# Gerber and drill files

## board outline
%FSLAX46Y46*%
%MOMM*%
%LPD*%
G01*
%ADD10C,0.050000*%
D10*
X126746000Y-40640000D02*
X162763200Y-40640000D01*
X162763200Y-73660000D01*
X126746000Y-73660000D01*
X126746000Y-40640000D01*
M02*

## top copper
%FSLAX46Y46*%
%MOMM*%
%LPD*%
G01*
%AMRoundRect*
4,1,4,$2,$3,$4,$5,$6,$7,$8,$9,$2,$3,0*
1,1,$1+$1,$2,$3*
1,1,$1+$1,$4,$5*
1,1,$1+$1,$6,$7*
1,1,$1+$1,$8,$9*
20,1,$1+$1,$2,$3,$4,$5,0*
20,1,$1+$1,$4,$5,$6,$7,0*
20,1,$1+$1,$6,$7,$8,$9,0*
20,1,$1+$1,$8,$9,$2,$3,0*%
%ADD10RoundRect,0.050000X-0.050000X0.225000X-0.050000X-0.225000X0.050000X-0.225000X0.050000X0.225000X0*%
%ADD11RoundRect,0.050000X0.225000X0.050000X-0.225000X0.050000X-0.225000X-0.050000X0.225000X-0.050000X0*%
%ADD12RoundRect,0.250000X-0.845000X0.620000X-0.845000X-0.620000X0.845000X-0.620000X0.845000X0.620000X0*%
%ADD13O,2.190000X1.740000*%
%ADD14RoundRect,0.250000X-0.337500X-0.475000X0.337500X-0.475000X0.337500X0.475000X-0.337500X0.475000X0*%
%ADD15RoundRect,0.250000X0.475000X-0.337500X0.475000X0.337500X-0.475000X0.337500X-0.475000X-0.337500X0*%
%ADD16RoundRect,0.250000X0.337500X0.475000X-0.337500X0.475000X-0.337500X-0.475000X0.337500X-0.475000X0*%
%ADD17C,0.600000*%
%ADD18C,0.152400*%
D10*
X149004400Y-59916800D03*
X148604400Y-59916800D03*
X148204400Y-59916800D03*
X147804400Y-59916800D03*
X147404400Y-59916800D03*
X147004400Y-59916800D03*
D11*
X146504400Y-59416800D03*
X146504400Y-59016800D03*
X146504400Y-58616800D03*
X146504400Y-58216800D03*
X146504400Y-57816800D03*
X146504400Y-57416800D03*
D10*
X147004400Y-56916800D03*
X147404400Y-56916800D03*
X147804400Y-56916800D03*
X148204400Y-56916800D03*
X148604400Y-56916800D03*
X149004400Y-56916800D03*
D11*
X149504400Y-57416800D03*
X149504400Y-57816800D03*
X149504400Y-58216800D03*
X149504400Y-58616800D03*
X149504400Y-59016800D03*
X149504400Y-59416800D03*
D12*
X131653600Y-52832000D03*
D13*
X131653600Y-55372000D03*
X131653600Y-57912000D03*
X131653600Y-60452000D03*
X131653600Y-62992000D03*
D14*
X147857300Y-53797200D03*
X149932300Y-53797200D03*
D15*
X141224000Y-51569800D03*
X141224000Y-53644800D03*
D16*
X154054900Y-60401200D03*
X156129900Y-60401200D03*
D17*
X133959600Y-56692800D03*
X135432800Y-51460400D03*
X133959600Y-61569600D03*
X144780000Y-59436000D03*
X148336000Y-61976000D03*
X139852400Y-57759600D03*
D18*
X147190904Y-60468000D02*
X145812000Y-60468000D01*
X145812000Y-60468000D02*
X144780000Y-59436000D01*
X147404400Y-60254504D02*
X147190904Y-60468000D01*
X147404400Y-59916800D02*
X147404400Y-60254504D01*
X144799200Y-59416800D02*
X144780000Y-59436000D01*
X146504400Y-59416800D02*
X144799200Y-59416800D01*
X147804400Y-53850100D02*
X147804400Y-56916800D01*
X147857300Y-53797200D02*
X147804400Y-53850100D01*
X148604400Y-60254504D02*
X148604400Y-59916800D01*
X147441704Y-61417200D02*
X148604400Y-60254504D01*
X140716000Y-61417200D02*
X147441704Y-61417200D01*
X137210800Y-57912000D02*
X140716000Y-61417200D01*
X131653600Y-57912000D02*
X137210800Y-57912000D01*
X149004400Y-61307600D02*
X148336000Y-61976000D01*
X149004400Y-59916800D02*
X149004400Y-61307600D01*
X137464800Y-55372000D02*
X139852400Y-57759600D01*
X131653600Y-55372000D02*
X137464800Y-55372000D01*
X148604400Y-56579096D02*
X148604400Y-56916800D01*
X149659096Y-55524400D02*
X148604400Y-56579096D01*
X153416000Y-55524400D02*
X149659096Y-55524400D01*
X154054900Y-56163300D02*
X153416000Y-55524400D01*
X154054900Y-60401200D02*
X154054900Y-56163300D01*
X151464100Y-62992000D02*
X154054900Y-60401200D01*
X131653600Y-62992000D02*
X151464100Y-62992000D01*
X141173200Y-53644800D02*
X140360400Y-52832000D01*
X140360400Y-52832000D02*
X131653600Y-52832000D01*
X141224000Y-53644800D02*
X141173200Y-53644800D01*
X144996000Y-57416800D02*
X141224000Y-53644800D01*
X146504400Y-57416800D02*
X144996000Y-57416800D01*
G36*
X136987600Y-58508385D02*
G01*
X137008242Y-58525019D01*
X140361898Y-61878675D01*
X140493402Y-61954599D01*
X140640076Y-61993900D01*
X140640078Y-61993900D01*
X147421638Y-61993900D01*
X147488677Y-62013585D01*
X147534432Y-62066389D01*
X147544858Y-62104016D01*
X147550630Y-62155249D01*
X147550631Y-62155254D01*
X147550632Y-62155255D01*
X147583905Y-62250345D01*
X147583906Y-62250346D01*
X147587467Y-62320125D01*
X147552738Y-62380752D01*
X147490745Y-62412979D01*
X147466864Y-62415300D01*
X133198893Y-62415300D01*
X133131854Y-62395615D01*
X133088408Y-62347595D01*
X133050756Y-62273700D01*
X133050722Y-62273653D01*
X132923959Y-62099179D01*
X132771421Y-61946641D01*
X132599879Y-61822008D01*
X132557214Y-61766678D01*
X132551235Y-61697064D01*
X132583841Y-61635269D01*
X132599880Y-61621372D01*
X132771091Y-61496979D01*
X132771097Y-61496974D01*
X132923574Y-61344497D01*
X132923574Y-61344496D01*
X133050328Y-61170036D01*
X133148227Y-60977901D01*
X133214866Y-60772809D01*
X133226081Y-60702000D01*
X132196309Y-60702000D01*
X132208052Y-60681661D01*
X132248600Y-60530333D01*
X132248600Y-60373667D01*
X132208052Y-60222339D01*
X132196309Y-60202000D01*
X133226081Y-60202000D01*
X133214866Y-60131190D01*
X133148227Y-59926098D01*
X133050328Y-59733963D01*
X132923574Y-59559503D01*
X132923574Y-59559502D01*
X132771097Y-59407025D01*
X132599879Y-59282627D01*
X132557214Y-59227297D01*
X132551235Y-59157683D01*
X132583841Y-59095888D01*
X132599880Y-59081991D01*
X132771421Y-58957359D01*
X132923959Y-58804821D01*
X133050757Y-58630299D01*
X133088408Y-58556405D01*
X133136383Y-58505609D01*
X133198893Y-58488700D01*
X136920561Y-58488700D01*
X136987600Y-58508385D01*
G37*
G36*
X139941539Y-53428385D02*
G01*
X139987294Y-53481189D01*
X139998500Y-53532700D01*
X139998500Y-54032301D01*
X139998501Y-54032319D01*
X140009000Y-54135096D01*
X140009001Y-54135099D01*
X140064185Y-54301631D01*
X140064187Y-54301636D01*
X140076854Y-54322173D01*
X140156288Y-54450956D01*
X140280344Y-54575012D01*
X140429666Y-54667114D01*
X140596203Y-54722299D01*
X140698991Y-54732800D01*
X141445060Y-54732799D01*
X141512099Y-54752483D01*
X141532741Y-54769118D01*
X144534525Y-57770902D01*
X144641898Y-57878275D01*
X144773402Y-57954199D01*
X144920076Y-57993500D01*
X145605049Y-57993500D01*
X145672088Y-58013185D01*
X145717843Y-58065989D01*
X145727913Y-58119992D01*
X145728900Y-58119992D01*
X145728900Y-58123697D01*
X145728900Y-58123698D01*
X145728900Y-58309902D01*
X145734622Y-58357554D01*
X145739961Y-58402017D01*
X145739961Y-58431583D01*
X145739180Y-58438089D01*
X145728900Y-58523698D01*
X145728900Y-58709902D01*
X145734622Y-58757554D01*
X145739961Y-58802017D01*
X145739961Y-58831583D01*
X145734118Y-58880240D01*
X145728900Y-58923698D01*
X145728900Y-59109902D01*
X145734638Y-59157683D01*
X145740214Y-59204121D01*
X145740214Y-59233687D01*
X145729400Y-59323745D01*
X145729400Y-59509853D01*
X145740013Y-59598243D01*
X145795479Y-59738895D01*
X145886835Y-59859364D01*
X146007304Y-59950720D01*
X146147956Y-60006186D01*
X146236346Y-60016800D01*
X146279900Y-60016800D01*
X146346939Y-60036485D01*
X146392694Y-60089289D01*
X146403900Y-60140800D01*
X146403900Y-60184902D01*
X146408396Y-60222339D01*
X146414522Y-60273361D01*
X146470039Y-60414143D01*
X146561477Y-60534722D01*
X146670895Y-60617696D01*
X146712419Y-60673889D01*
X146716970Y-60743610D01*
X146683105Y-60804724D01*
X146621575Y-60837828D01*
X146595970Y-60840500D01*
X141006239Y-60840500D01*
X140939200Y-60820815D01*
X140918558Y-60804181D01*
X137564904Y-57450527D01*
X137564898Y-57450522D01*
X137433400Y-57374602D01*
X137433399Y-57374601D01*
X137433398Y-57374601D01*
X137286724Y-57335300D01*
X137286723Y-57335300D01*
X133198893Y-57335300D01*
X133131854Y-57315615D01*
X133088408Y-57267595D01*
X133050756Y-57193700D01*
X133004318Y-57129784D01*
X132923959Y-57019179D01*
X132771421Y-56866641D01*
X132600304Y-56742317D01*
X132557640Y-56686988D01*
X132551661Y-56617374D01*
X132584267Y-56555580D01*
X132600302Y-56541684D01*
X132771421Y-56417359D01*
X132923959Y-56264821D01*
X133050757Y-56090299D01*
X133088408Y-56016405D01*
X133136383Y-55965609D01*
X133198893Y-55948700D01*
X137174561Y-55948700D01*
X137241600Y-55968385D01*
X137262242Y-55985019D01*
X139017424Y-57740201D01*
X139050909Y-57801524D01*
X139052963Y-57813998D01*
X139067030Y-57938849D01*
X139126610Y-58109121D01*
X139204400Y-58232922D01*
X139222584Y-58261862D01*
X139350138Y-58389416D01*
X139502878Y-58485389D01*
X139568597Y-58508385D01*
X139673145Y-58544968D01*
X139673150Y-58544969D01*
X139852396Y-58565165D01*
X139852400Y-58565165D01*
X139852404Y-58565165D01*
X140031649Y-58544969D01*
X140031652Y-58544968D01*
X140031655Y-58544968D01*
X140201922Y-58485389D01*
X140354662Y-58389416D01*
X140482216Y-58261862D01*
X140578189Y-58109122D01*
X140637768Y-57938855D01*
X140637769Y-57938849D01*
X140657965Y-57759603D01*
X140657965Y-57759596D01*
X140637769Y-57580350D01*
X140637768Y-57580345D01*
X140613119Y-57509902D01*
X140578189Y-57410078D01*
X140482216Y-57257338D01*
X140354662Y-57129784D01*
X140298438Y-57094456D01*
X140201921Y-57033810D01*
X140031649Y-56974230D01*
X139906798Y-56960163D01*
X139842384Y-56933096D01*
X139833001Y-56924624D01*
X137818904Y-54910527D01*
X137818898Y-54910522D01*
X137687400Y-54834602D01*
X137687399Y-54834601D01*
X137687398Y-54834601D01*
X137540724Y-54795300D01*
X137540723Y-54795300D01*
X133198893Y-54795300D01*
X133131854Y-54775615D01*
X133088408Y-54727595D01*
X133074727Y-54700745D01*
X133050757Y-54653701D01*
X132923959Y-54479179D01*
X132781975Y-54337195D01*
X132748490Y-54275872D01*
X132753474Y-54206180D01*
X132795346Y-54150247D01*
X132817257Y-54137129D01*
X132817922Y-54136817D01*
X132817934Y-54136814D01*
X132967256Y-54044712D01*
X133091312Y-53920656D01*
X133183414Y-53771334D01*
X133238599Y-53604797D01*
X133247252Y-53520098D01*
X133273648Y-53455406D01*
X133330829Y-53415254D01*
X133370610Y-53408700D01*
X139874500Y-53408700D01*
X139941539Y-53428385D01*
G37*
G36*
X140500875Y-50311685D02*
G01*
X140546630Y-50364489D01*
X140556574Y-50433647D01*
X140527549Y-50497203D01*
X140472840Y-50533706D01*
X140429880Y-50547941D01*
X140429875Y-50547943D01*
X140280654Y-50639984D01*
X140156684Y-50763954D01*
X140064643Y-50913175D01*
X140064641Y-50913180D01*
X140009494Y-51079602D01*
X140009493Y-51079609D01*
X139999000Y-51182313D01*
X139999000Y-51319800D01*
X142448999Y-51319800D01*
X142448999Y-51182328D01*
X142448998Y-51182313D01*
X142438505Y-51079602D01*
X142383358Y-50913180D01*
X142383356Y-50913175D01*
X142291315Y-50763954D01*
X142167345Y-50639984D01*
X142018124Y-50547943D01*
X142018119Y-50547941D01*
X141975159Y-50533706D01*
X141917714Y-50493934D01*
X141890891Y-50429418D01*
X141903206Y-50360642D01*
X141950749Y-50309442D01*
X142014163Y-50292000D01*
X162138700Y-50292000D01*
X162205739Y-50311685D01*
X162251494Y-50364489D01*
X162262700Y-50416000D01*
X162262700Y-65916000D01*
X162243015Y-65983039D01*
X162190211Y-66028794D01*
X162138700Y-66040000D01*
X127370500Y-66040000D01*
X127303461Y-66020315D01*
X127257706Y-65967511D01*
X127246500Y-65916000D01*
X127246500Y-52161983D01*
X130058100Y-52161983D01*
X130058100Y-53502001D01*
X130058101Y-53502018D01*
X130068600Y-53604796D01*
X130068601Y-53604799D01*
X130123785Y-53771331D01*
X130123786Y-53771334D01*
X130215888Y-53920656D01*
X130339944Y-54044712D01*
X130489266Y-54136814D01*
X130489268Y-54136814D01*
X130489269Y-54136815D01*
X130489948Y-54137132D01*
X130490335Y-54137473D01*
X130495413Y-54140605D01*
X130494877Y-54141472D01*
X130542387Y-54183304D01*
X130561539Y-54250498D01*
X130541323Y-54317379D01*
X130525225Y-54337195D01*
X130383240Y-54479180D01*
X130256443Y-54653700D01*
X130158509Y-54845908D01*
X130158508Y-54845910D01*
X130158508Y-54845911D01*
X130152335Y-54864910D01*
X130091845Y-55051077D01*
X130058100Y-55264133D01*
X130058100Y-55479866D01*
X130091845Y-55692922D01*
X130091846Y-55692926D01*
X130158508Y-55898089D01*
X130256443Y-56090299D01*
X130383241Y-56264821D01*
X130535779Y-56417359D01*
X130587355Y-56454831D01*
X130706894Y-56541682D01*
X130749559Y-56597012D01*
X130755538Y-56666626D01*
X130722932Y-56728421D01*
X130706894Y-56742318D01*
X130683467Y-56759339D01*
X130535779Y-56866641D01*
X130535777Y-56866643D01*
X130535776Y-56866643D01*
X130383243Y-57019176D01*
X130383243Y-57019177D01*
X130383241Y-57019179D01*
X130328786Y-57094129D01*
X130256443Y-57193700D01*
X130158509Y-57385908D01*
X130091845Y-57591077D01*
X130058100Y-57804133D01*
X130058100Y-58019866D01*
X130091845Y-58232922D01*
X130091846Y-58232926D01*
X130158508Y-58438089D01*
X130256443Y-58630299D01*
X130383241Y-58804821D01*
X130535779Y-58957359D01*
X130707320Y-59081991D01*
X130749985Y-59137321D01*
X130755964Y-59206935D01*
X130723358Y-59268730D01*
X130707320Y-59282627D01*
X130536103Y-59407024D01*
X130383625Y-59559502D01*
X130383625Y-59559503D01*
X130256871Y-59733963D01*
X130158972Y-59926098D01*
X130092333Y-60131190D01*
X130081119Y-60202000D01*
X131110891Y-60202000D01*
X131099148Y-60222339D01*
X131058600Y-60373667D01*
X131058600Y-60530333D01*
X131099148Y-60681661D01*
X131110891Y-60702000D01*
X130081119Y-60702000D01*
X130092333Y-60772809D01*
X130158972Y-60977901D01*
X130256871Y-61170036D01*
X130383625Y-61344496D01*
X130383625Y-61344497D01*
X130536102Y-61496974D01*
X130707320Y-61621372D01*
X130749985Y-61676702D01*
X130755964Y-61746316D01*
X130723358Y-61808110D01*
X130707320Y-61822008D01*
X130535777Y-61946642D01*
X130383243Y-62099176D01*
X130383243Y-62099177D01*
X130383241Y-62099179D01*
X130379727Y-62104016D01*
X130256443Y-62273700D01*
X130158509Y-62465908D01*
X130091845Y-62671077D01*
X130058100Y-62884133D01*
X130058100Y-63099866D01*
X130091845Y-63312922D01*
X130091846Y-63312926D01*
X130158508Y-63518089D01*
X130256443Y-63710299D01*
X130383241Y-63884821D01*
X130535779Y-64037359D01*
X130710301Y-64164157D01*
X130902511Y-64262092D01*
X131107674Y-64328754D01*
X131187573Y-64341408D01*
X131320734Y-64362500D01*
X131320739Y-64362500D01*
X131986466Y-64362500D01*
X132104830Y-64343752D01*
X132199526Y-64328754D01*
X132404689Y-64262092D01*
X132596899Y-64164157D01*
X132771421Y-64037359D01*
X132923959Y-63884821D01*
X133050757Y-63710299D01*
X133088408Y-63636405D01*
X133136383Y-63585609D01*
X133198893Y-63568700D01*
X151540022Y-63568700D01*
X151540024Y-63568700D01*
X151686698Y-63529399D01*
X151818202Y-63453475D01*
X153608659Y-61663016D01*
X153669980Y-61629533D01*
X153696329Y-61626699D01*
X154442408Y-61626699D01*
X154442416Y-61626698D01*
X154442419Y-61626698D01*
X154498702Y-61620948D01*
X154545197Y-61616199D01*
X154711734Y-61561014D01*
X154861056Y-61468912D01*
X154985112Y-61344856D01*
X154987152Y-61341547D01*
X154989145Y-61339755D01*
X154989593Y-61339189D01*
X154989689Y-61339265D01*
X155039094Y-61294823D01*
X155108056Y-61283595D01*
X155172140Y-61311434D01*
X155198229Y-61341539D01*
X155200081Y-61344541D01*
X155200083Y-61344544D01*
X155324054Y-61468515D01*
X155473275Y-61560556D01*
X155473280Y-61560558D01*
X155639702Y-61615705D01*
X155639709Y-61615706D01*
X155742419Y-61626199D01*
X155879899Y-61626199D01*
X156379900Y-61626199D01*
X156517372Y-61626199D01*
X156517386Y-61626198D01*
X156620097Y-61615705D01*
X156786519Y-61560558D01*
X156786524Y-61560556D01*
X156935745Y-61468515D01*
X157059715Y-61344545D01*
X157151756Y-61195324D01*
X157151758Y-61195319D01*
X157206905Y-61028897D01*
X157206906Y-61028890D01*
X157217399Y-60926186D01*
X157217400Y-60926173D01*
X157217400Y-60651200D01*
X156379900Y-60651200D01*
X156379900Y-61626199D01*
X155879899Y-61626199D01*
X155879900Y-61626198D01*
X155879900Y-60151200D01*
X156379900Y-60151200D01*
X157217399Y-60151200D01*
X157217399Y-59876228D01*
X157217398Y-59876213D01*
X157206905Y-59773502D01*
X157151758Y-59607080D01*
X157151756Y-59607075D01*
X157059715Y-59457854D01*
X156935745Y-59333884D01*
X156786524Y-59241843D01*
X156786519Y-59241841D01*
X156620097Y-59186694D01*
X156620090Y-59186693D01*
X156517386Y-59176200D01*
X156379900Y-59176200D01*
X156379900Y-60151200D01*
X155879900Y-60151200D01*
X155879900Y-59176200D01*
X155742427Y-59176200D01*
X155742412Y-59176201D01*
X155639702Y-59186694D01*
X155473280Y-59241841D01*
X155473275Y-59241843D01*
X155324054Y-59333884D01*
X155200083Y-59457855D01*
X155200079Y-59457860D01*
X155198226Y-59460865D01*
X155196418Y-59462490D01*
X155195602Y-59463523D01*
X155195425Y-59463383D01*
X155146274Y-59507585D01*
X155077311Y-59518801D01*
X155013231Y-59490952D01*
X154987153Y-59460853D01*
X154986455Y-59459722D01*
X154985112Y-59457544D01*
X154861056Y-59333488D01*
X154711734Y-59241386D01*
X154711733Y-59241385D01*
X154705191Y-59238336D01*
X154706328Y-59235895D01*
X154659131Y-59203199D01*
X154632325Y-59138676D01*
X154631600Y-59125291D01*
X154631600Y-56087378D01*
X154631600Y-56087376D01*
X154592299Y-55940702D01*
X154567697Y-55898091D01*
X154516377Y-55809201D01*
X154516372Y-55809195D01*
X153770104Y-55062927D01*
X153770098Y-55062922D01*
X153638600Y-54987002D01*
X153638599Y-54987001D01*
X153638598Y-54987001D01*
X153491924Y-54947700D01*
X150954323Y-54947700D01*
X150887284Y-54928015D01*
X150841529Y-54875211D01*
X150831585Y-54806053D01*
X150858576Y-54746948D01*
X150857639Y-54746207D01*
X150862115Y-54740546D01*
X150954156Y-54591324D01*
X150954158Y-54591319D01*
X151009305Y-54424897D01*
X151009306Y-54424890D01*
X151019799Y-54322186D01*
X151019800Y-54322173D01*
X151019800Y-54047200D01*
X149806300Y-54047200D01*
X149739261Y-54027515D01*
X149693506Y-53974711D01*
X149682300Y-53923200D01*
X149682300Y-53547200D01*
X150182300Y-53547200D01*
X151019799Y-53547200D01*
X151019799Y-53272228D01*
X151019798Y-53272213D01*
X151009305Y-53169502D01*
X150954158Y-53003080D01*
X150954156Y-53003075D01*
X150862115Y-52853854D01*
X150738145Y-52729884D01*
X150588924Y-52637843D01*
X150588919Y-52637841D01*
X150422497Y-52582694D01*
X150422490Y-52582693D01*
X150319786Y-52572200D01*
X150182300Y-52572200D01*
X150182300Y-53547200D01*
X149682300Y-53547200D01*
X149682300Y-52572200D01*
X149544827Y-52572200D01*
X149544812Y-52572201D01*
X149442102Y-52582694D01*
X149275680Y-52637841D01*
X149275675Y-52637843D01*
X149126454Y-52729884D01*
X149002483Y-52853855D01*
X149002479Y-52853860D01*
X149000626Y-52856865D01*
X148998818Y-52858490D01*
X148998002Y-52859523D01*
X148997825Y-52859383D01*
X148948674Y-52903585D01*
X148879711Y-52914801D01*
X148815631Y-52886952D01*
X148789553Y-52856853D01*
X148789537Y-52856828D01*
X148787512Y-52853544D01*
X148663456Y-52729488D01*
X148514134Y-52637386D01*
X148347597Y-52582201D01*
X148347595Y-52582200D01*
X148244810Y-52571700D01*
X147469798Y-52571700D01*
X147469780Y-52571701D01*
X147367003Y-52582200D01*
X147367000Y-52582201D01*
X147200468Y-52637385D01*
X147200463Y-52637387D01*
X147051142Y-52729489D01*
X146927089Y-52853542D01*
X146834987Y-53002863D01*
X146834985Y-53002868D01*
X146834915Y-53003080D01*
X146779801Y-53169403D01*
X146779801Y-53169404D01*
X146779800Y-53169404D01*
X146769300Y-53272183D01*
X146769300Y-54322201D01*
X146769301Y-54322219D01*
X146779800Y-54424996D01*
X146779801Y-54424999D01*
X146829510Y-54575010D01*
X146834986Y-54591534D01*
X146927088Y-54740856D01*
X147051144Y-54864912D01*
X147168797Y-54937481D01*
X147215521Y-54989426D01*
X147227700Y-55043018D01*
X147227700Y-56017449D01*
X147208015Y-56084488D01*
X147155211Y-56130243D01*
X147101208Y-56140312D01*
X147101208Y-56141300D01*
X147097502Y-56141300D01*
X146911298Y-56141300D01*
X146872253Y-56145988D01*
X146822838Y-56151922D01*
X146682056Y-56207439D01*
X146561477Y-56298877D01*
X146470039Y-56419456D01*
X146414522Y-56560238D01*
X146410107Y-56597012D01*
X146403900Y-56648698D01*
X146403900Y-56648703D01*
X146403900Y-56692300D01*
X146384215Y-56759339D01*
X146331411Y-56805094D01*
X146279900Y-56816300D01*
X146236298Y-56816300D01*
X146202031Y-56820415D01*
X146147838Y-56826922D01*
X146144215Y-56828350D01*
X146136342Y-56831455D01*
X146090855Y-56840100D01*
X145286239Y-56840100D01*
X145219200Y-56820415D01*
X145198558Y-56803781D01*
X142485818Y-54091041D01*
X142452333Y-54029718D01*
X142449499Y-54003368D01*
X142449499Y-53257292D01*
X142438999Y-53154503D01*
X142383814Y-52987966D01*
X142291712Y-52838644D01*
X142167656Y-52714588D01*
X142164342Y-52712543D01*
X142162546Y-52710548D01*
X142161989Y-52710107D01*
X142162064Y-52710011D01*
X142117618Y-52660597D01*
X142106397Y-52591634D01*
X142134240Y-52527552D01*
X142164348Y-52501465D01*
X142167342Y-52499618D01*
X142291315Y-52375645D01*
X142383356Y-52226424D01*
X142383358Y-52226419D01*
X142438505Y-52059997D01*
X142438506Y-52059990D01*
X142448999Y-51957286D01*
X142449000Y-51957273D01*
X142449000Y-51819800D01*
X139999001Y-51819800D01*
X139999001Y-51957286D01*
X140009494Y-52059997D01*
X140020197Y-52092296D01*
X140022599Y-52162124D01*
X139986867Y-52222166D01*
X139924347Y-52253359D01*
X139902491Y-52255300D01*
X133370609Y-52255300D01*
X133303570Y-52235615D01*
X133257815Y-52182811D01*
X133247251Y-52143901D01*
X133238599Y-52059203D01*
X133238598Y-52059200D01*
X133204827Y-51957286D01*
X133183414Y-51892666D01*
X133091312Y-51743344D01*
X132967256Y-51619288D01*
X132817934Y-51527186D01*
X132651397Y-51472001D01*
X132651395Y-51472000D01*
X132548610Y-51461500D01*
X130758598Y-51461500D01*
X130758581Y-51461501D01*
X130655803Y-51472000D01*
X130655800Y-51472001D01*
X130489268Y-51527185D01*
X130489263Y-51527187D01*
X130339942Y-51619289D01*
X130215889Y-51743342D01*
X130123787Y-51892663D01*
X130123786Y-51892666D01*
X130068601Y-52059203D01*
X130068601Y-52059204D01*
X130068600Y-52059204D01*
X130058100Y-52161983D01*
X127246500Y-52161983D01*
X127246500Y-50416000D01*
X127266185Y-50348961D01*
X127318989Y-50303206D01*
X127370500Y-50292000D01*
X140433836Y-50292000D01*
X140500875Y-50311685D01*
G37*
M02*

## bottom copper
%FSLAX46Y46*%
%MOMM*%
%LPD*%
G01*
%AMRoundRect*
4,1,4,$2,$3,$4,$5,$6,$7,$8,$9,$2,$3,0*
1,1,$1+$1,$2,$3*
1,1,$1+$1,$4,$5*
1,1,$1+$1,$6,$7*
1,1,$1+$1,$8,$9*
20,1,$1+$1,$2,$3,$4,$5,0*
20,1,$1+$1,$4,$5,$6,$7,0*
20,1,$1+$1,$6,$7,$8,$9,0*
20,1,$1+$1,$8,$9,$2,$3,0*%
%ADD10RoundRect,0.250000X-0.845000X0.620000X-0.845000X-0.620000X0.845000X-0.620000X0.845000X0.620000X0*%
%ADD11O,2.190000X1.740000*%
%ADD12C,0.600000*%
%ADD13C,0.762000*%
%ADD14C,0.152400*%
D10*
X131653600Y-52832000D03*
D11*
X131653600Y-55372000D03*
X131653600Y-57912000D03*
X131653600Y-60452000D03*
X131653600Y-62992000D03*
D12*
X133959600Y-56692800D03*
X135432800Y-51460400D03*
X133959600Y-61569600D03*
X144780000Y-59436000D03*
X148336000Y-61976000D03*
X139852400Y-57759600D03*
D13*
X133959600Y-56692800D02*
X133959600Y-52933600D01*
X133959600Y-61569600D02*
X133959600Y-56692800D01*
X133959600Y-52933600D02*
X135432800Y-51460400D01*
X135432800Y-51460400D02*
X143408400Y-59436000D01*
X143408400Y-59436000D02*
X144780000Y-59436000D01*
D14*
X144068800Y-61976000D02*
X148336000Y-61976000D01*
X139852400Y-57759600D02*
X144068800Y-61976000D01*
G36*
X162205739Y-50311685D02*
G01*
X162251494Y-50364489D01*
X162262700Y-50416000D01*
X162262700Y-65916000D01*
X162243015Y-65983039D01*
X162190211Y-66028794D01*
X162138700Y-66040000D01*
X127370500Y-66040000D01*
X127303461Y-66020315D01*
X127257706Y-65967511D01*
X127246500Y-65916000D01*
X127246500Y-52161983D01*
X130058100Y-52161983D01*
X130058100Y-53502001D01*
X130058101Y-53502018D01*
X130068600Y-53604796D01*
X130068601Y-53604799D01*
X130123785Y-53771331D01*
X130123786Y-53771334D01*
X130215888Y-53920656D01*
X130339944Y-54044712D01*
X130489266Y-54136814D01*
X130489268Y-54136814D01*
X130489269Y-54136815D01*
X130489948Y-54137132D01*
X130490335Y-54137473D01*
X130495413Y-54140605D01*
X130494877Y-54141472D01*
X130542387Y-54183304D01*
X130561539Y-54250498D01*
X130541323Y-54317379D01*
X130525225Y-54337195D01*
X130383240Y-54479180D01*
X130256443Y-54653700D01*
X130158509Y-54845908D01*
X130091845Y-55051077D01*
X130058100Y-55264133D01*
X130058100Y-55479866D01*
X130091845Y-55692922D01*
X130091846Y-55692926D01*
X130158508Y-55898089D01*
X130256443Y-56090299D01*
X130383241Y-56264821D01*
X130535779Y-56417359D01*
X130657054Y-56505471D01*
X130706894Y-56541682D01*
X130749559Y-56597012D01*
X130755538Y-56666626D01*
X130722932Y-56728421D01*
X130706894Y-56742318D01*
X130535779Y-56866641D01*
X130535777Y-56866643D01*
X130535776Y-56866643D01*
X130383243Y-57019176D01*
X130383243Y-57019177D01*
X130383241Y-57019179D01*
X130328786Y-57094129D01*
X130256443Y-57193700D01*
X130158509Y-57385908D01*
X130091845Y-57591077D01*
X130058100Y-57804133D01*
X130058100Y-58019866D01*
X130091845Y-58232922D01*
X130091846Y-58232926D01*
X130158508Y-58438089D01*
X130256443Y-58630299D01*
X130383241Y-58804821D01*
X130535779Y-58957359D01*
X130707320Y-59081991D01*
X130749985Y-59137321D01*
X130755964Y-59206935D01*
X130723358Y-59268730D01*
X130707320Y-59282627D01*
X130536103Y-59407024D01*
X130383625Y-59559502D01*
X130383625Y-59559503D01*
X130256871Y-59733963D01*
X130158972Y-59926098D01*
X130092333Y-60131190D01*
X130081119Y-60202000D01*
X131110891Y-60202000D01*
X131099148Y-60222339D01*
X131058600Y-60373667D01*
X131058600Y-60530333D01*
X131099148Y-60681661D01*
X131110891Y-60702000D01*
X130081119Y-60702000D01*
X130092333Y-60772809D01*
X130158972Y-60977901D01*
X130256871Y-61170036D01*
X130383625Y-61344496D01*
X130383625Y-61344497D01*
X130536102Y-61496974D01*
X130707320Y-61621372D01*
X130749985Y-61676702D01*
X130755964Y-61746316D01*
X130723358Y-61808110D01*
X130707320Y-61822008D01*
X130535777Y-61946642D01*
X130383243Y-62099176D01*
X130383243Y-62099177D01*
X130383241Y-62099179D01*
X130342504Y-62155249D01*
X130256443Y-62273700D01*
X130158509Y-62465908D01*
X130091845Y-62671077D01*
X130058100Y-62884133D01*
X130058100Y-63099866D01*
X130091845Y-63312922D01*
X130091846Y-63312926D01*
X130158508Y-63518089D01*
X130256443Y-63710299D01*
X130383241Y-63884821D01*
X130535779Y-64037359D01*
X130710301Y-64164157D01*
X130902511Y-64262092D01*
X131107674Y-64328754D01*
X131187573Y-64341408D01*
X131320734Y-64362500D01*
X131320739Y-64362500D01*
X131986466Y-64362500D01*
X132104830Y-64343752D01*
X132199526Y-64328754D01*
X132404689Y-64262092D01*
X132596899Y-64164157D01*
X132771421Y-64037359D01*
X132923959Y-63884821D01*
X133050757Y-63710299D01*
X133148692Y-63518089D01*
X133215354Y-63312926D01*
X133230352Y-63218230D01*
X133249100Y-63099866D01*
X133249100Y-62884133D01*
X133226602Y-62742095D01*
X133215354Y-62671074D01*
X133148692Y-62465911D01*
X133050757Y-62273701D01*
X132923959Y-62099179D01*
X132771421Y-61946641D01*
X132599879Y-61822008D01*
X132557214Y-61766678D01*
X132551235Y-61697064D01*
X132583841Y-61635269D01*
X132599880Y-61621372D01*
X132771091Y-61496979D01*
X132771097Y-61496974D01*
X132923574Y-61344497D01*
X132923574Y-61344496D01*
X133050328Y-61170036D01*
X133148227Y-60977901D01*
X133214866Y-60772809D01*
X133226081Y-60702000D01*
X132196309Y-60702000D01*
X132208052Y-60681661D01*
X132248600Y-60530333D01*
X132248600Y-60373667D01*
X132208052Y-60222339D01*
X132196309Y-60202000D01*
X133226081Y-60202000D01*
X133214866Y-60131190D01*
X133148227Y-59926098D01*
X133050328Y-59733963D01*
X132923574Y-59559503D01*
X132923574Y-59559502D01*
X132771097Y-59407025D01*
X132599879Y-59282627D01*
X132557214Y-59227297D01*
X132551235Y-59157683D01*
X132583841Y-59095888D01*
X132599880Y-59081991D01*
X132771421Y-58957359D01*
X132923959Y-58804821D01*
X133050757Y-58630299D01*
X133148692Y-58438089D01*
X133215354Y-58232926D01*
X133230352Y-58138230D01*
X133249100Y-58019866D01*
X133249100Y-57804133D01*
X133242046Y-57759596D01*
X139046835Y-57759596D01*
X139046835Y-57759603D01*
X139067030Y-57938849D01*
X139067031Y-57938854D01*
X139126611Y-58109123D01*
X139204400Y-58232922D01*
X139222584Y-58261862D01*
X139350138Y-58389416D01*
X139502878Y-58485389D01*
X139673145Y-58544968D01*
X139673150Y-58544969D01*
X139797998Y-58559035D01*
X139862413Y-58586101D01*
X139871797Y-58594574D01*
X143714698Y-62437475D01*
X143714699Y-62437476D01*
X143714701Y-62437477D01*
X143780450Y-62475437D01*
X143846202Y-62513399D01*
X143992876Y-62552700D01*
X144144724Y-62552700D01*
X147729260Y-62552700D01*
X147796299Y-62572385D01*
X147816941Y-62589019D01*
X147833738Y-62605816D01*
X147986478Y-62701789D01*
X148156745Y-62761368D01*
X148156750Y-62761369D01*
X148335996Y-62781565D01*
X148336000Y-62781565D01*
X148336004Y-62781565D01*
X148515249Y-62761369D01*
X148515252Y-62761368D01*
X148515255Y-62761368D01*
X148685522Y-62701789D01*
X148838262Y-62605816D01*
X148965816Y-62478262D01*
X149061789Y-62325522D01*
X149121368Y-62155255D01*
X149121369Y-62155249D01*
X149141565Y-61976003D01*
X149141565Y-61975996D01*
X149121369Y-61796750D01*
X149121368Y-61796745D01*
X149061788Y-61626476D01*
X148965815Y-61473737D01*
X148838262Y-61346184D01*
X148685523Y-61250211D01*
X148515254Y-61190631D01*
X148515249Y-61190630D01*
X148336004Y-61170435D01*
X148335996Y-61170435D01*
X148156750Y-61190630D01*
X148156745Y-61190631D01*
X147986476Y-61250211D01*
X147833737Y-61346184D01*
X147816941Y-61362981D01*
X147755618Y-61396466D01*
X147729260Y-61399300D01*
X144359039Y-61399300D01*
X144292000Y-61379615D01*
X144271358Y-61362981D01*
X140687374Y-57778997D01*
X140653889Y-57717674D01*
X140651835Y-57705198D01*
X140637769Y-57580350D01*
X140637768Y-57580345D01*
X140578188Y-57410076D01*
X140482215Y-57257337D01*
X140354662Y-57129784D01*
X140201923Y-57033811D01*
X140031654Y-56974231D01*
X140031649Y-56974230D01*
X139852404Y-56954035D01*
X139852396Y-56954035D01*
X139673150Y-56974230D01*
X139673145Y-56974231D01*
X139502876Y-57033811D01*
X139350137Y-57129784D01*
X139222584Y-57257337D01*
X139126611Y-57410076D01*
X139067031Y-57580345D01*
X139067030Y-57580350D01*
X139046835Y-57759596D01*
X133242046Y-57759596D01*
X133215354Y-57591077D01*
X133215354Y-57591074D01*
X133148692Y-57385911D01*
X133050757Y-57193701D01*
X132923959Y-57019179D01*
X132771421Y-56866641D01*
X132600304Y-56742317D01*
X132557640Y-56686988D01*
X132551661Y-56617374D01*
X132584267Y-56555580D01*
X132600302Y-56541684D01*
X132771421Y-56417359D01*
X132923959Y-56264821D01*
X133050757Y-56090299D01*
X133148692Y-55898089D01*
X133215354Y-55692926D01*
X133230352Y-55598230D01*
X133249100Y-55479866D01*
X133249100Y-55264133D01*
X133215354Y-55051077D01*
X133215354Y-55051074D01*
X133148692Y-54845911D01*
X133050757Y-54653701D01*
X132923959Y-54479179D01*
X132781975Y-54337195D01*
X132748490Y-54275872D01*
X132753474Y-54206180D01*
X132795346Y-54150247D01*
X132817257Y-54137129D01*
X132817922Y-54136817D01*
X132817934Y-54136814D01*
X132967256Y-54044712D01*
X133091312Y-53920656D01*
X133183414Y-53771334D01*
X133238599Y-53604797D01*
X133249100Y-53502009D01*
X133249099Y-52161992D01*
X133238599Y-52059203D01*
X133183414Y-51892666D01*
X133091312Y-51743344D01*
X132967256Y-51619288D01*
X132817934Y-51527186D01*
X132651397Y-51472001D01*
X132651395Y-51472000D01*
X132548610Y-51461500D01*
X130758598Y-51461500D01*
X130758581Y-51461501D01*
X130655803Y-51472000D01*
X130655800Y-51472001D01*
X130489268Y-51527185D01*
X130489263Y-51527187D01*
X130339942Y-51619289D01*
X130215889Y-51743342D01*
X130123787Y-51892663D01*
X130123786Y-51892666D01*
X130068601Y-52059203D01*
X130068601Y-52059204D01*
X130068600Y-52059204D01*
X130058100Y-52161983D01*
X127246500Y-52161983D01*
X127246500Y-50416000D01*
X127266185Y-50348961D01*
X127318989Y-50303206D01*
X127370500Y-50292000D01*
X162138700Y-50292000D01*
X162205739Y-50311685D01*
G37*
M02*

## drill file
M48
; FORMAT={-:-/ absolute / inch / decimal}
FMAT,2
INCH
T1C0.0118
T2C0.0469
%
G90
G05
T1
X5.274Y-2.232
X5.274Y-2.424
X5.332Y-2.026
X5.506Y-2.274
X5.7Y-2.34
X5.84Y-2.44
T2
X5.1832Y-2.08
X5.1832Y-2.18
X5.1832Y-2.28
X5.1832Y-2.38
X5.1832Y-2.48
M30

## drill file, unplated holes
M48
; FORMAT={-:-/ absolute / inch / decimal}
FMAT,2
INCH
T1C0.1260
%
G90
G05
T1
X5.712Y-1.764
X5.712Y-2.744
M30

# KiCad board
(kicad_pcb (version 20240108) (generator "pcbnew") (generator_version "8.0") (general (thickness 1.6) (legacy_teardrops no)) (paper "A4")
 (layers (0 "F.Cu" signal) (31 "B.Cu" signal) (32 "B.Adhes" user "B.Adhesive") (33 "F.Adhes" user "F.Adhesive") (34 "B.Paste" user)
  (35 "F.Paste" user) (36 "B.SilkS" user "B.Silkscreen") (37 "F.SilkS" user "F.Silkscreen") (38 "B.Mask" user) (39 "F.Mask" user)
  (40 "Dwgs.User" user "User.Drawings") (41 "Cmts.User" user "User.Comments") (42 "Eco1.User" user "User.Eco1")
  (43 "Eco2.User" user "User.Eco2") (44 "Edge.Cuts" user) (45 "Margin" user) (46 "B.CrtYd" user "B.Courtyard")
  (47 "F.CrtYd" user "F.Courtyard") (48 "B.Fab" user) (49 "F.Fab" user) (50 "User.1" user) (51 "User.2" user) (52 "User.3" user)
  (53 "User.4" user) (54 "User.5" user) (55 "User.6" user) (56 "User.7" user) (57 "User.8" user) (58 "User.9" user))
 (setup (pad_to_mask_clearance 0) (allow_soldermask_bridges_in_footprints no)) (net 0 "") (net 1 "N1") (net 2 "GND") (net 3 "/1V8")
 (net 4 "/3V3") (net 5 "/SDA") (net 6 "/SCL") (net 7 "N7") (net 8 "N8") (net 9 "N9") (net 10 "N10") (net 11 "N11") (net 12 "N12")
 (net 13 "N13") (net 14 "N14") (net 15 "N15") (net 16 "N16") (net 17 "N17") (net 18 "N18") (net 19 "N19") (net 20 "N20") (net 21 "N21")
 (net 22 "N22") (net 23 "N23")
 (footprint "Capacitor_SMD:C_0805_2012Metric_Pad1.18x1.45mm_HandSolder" (layer "F.Cu") (at 148.8948 53.7972)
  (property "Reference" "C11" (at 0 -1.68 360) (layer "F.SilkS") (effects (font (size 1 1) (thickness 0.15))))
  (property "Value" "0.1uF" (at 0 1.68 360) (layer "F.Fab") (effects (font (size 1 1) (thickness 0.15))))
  (pad "1" smd roundrect (at -1.0375 0) (size 1.175 1.45) (layers "F.Cu" "F.Paste" "F.Mask") (roundrect_rratio 0.212766) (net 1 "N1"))
  (pad "2" smd roundrect (at 1.0375 0) (size 1.175 1.45) (layers "F.Cu" "F.Paste" "F.Mask") (roundrect_rratio 0.212766) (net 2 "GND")))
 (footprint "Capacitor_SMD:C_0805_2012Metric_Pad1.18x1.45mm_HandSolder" (layer "F.Cu") (at 155.0924 60.4012 180)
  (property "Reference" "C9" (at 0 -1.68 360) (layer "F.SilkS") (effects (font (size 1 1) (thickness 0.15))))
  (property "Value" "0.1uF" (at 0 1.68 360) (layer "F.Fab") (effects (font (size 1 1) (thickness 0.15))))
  (pad "1" smd roundrect (at -1.0375 0 180) (size 1.175 1.45) (layers "F.Cu" "F.Paste" "F.Mask") (roundrect_rratio 0.212766) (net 2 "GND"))
  (pad "2" smd roundrect (at 1.0375 0 180) (size 1.175 1.45) (layers "F.Cu" "F.Paste" "F.Mask") (roundrect_rratio 0.212766) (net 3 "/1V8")))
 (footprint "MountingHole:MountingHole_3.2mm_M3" (layer "F.Cu") (at 145.0848 69.6976)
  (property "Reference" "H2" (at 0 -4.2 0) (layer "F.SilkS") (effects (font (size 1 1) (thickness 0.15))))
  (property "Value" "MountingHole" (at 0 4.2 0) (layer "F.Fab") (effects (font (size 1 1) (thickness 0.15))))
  (pad "" np_thru_hole circle (at 0 0) (size 3.2 3.2) (drill 3.2) (layers "*.Cu" "*.Mask")))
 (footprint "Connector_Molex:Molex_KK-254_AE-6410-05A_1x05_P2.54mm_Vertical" (layer "F.Cu") (at 131.6536 52.832 -90)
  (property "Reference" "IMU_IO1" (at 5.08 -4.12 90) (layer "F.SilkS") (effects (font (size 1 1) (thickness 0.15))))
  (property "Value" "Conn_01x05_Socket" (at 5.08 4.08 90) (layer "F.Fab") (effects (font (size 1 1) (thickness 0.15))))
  (pad "1" thru_hole roundrect (at 0 0 270) (size 1.74 2.19) (drill 1.19) (layers "*.Cu" "*.Mask") (remove_unused_layers no)
   (roundrect_rratio 0.143678) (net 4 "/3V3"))
  (pad "2" thru_hole oval (at 2.54 0 270) (size 1.74 2.19) (drill 1.19) (layers "*.Cu" "*.Mask") (remove_unused_layers no) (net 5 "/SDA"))
  (pad "3" thru_hole oval (at 5.08 0 270) (size 1.74 2.19) (drill 1.19) (layers "*.Cu" "*.Mask") (remove_unused_layers no) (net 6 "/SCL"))
  (pad "4" thru_hole oval (at 7.62 0 270) (size 1.74 2.19) (drill 1.19) (layers "*.Cu" "*.Mask") (remove_unused_layers no) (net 2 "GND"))
  (pad "5" thru_hole oval (at 10.16 0 270) (size 1.74 2.19) (drill 1.19) (layers "*.Cu" "*.Mask") (remove_unused_layers no) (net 3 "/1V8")))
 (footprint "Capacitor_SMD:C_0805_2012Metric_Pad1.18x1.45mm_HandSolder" (layer "F.Cu") (at 141.224 52.6073 90)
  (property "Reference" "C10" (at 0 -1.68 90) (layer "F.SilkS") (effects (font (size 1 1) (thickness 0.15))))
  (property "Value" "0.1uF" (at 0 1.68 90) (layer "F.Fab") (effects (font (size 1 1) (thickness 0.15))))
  (pad "1" smd roundrect (at -1.0375 0 90) (size 1.175 1.45) (layers "F.Cu" "F.Paste" "F.Mask") (roundrect_rratio 0.212766) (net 4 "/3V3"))
  (pad "2" smd roundrect (at 1.0375 0 90) (size 1.175 1.45) (layers "F.Cu" "F.Paste" "F.Mask") (roundrect_rratio 0.212766) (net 2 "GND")))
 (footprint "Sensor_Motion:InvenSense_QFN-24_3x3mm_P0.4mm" (layer "F.Cu") (at 148.0044 58.4168 180)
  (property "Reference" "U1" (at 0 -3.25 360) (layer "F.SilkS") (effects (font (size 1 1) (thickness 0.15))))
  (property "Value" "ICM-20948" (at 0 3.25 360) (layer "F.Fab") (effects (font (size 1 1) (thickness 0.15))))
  (pad "1" smd roundrect (at -1.5 -1 180) (size 0.55 0.2) (layers "F.Cu" "F.Paste" "F.Mask") (roundrect_rratio 0.25) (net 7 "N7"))
  (pad "2" smd roundrect (at -1.5 -0.6 180) (size 0.55 0.2) (layers "F.Cu" "F.Paste" "F.Mask") (roundrect_rratio 0.25) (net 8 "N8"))
  (pad "3" smd roundrect (at -1.5 -0.2 180) (size 0.55 0.2) (layers "F.Cu" "F.Paste" "F.Mask") (roundrect_rratio 0.25) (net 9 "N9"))
  (pad "4" smd roundrect (at -1.5 0.2 180) (size 0.55 0.2) (layers "F.Cu" "F.Paste" "F.Mask") (roundrect_rratio 0.25) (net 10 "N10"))
  (pad "5" smd roundrect (at -1.5 0.6 180) (size 0.55 0.2) (layers "F.Cu" "F.Paste" "F.Mask") (roundrect_rratio 0.25) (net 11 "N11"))
  (pad "6" smd roundrect (at -1.5 1 180) (size 0.55 0.2) (layers "F.Cu" "F.Paste" "F.Mask") (roundrect_rratio 0.25) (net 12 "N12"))
  (pad "7" smd roundrect (at -1 1.5 270) (size 0.55 0.2) (layers "F.Cu" "F.Paste" "F.Mask") (roundrect_rratio 0.25) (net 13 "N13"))
  (pad "8" smd roundrect (at -0.6 1.5 270) (size 0.55 0.2) (layers "F.Cu" "F.Paste" "F.Mask") (roundrect_rratio 0.25) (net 3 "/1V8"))
  (pad "9" smd roundrect (at -0.2 1.5 270) (size 0.55 0.2) (layers "F.Cu" "F.Paste" "F.Mask") (roundrect_rratio 0.25) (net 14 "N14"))
  (pad "10" smd roundrect (at 0.2 1.5 270) (size 0.55 0.2) (layers "F.Cu" "F.Paste" "F.Mask") (roundrect_rratio 0.25) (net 1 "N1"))
  (pad "11" smd roundrect (at 0.6 1.5 270) (size 0.55 0.2) (layers "F.Cu" "F.Paste" "F.Mask") (roundrect_rratio 0.25) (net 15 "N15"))
  (pad "12" smd roundrect (at 1 1.5 270) (size 0.55 0.2) (layers "F.Cu" "F.Paste" "F.Mask") (roundrect_rratio 0.25) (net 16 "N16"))
  (pad "13" smd roundrect (at 1.5 1 180) (size 0.55 0.2) (layers "F.Cu" "F.Paste" "F.Mask") (roundrect_rratio 0.25) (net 4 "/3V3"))
  (pad "14" smd roundrect (at 1.5 0.6 180) (size 0.55 0.2) (layers "F.Cu" "F.Paste" "F.Mask") (roundrect_rratio 0.25) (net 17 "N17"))
  (pad "15" smd roundrect (at 1.5 0.2 180) (size 0.55 0.2) (layers "F.Cu" "F.Paste" "F.Mask") (roundrect_rratio 0.25) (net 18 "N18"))
  (pad "16" smd roundrect (at 1.5 -0.2 180) (size 0.55 0.2) (layers "F.Cu" "F.Paste" "F.Mask") (roundrect_rratio 0.25) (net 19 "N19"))
  (pad "17" smd roundrect (at 1.5 -0.6 180) (size 0.55 0.2) (layers "F.Cu" "F.Paste" "F.Mask") (roundrect_rratio 0.25) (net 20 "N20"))
  (pad "18" smd roundrect (at 1.5 -1 180) (size 0.55 0.2) (layers "F.Cu" "F.Paste" "F.Mask") (roundrect_rratio 0.25) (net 2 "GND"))
  (pad "19" smd roundrect (at 1 -1.5 270) (size 0.55 0.2) (layers "F.Cu" "F.Paste" "F.Mask") (roundrect_rratio 0.25) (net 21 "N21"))
  (pad "20" smd roundrect (at 0.6 -1.5 270) (size 0.55 0.2) (layers "F.Cu" "F.Paste" "F.Mask") (roundrect_rratio 0.25) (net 2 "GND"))
  (pad "21" smd roundrect (at 0.2 -1.5 270) (size 0.55 0.2) (layers "F.Cu" "F.Paste" "F.Mask") (roundrect_rratio 0.25) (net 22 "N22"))
  (pad "22" smd roundrect (at -0.2 -1.5 270) (size 0.55 0.2) (layers "F.Cu" "F.Paste" "F.Mask") (roundrect_rratio 0.25) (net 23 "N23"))
  (pad "23" smd roundrect (at -0.6 -1.5 270) (size 0.55 0.2) (layers "F.Cu" "F.Paste" "F.Mask") (roundrect_rratio 0.25) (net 6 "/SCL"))
  (pad "24" smd roundrect (at -1 -1.5 270) (size 0.55 0.2) (layers "F.Cu" "F.Paste" "F.Mask") (roundrect_rratio 0.25) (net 5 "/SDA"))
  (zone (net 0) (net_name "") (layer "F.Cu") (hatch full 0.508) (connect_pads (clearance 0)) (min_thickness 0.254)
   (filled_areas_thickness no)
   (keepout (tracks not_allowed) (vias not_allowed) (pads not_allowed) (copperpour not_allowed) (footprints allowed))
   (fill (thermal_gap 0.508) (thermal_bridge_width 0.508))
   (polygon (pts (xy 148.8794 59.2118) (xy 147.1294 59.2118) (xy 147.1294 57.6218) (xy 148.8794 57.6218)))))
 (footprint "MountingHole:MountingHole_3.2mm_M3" (layer "F.Cu") (at 145.0848 44.8056)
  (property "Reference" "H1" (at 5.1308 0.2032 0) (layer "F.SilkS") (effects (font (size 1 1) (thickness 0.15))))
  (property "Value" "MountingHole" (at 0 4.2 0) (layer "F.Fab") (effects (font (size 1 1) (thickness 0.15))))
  (pad "" np_thru_hole circle (at 0 0) (size 3.2 3.2) (drill 3.2) (layers "*.Cu" "*.Mask")))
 (gr_rect (start 126.746 40.64) (end 162.7632 73.66) (stroke (width 0.05) (type default)) (fill none) (layer "Edge.Cuts"))
 (segment (start 148.6044 56.579096) (end 148.6044 56.9168) (width 0.1524) (layer "F.Cu") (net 3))
 (segment (start 131.6536 62.992) (end 151.4641 62.992) (width 0.1524) (layer "F.Cu") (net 3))
 (segment (start 154.0549 56.1633) (end 153.416 55.5244) (width 0.1524) (layer "F.Cu") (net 3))
 (segment (start 149.659096 55.5244) (end 148.6044 56.579096) (width 0.1524) (layer "F.Cu") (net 3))
 (segment (start 153.416 55.5244) (end 149.659096 55.5244) (width 0.1524) (layer "F.Cu") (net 3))
 (segment (start 154.0549 60.4012) (end 154.0549 56.1633) (width 0.1524) (layer "F.Cu") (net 3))
 (segment (start 151.4641 62.992) (end 154.0549 60.4012) (width 0.1524) (layer "F.Cu") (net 3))
 (segment (start 146.5044 59.4168) (end 144.7992 59.4168) (width 0.1524) (layer "F.Cu") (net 2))
 (segment (start 145.812 60.468) (end 144.78 59.436) (width 0.1524) (layer "F.Cu") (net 2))
 (segment (start 144.7992 59.4168) (end 144.78 59.436) (width 0.1524) (layer "F.Cu") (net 2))
 (segment (start 147.4044 60.254504) (end 147.190904 60.468) (width 0.1524) (layer "F.Cu") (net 2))
 (segment (start 147.4044 59.9168) (end 147.4044 60.254504) (width 0.1524) (layer "F.Cu") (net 2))
 (segment (start 147.190904 60.468) (end 145.812 60.468) (width 0.1524) (layer "F.Cu") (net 2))
 (via (at 144.78 59.436) (size 0.6) (drill 0.3) (layers "F.Cu" "B.Cu") (free yes) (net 2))
 (via (at 133.9596 61.5696) (size 0.6) (drill 0.3) (layers "F.Cu" "B.Cu") (free yes) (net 2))
 (via (at 133.9596 56.6928) (size 0.6) (drill 0.3) (layers "F.Cu" "B.Cu") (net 2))
 (via (at 135.4328 51.4604) (size 0.6) (drill 0.3) (layers "F.Cu" "B.Cu") (free yes) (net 2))
 (segment (start 133.9596 61.5696) (end 133.9596 56.6928) (width 0.762) (layer "B.Cu") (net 2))
 (segment (start 133.9596 52.9336) (end 135.4328 51.4604) (width 0.762) (layer "B.Cu") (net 2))
 (segment (start 143.4084 59.436) (end 144.78 59.436) (width 0.762) (layer "B.Cu") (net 2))
 (segment (start 133.9596 56.6928) (end 133.9596 52.9336) (width 0.762) (layer "B.Cu") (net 2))
 (segment (start 135.4328 51.4604) (end 143.4084 59.436) (width 0.762) (layer "B.Cu") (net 2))
 (segment (start 141.1732 53.6448) (end 140.3604 52.832) (width 0.1524) (layer "F.Cu") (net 4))
 (segment (start 140.3604 52.832) (end 131.6536 52.832) (width 0.1524) (layer "F.Cu") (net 4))
 (segment (start 144.996 57.4168) (end 141.224 53.6448) (width 0.1524) (layer "F.Cu") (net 4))
 (segment (start 146.5044 57.4168) (end 144.996 57.4168) (width 0.1524) (layer "F.Cu") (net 4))
 (segment (start 141.224 53.6448) (end 141.1732 53.6448) (width 0.1524) (layer "F.Cu") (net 4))
 (segment (start 147.8044 53.8501) (end 147.8044 56.9168) (width 0.1524) (layer "F.Cu") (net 1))
 (segment (start 147.8573 53.7972) (end 147.8044 53.8501) (width 0.1524) (layer "F.Cu") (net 1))
 (segment (start 149.0044 61.3076) (end 148.336 61.976) (width 0.1524) (layer "F.Cu") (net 5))
 (segment (start 137.4648 55.372) (end 139.8524 57.7596) (width 0.1524) (layer "F.Cu") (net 5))
 (segment (start 131.6536 55.372) (end 137.4648 55.372) (width 0.1524) (layer "F.Cu") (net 5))
 (segment (start 149.0044 59.9168) (end 149.0044 61.3076) (width 0.1524) (layer "F.Cu") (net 5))
 (via (at 148.336 61.976) (size 0.6) (drill 0.3) (layers "F.Cu" "B.Cu") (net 5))
 (via (at 139.8524 57.7596) (size 0.6) (drill 0.3) (layers "F.Cu" "B.Cu") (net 5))
 (segment (start 139.8524 57.7596) (end 144.0688 61.976) (width 0.1524) (layer "B.Cu") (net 5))
 (segment (start 144.0688 61.976) (end 148.336 61.976) (width 0.1524) (layer "B.Cu") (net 5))
 (segment (start 131.6536 57.912) (end 137.2108 57.912) (width 0.1524) (layer "F.Cu") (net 6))
 (segment (start 147.441704 61.4172) (end 148.6044 60.254504) (width 0.1524) (layer "F.Cu") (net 6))
 (segment (start 148.6044 60.254504) (end 148.6044 59.9168) (width 0.1524) (layer "F.Cu") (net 6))
 (segment (start 137.2108 57.912) (end 140.716 61.4172) (width 0.1524) (layer "F.Cu") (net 6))
 (segment (start 140.716 61.4172) (end 147.441704 61.4172) (width 0.1524) (layer "F.Cu") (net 6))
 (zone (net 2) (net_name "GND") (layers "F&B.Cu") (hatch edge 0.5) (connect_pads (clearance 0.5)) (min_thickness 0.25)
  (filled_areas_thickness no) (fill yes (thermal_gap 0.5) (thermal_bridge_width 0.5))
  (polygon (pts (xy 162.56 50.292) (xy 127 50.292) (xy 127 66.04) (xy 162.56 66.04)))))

